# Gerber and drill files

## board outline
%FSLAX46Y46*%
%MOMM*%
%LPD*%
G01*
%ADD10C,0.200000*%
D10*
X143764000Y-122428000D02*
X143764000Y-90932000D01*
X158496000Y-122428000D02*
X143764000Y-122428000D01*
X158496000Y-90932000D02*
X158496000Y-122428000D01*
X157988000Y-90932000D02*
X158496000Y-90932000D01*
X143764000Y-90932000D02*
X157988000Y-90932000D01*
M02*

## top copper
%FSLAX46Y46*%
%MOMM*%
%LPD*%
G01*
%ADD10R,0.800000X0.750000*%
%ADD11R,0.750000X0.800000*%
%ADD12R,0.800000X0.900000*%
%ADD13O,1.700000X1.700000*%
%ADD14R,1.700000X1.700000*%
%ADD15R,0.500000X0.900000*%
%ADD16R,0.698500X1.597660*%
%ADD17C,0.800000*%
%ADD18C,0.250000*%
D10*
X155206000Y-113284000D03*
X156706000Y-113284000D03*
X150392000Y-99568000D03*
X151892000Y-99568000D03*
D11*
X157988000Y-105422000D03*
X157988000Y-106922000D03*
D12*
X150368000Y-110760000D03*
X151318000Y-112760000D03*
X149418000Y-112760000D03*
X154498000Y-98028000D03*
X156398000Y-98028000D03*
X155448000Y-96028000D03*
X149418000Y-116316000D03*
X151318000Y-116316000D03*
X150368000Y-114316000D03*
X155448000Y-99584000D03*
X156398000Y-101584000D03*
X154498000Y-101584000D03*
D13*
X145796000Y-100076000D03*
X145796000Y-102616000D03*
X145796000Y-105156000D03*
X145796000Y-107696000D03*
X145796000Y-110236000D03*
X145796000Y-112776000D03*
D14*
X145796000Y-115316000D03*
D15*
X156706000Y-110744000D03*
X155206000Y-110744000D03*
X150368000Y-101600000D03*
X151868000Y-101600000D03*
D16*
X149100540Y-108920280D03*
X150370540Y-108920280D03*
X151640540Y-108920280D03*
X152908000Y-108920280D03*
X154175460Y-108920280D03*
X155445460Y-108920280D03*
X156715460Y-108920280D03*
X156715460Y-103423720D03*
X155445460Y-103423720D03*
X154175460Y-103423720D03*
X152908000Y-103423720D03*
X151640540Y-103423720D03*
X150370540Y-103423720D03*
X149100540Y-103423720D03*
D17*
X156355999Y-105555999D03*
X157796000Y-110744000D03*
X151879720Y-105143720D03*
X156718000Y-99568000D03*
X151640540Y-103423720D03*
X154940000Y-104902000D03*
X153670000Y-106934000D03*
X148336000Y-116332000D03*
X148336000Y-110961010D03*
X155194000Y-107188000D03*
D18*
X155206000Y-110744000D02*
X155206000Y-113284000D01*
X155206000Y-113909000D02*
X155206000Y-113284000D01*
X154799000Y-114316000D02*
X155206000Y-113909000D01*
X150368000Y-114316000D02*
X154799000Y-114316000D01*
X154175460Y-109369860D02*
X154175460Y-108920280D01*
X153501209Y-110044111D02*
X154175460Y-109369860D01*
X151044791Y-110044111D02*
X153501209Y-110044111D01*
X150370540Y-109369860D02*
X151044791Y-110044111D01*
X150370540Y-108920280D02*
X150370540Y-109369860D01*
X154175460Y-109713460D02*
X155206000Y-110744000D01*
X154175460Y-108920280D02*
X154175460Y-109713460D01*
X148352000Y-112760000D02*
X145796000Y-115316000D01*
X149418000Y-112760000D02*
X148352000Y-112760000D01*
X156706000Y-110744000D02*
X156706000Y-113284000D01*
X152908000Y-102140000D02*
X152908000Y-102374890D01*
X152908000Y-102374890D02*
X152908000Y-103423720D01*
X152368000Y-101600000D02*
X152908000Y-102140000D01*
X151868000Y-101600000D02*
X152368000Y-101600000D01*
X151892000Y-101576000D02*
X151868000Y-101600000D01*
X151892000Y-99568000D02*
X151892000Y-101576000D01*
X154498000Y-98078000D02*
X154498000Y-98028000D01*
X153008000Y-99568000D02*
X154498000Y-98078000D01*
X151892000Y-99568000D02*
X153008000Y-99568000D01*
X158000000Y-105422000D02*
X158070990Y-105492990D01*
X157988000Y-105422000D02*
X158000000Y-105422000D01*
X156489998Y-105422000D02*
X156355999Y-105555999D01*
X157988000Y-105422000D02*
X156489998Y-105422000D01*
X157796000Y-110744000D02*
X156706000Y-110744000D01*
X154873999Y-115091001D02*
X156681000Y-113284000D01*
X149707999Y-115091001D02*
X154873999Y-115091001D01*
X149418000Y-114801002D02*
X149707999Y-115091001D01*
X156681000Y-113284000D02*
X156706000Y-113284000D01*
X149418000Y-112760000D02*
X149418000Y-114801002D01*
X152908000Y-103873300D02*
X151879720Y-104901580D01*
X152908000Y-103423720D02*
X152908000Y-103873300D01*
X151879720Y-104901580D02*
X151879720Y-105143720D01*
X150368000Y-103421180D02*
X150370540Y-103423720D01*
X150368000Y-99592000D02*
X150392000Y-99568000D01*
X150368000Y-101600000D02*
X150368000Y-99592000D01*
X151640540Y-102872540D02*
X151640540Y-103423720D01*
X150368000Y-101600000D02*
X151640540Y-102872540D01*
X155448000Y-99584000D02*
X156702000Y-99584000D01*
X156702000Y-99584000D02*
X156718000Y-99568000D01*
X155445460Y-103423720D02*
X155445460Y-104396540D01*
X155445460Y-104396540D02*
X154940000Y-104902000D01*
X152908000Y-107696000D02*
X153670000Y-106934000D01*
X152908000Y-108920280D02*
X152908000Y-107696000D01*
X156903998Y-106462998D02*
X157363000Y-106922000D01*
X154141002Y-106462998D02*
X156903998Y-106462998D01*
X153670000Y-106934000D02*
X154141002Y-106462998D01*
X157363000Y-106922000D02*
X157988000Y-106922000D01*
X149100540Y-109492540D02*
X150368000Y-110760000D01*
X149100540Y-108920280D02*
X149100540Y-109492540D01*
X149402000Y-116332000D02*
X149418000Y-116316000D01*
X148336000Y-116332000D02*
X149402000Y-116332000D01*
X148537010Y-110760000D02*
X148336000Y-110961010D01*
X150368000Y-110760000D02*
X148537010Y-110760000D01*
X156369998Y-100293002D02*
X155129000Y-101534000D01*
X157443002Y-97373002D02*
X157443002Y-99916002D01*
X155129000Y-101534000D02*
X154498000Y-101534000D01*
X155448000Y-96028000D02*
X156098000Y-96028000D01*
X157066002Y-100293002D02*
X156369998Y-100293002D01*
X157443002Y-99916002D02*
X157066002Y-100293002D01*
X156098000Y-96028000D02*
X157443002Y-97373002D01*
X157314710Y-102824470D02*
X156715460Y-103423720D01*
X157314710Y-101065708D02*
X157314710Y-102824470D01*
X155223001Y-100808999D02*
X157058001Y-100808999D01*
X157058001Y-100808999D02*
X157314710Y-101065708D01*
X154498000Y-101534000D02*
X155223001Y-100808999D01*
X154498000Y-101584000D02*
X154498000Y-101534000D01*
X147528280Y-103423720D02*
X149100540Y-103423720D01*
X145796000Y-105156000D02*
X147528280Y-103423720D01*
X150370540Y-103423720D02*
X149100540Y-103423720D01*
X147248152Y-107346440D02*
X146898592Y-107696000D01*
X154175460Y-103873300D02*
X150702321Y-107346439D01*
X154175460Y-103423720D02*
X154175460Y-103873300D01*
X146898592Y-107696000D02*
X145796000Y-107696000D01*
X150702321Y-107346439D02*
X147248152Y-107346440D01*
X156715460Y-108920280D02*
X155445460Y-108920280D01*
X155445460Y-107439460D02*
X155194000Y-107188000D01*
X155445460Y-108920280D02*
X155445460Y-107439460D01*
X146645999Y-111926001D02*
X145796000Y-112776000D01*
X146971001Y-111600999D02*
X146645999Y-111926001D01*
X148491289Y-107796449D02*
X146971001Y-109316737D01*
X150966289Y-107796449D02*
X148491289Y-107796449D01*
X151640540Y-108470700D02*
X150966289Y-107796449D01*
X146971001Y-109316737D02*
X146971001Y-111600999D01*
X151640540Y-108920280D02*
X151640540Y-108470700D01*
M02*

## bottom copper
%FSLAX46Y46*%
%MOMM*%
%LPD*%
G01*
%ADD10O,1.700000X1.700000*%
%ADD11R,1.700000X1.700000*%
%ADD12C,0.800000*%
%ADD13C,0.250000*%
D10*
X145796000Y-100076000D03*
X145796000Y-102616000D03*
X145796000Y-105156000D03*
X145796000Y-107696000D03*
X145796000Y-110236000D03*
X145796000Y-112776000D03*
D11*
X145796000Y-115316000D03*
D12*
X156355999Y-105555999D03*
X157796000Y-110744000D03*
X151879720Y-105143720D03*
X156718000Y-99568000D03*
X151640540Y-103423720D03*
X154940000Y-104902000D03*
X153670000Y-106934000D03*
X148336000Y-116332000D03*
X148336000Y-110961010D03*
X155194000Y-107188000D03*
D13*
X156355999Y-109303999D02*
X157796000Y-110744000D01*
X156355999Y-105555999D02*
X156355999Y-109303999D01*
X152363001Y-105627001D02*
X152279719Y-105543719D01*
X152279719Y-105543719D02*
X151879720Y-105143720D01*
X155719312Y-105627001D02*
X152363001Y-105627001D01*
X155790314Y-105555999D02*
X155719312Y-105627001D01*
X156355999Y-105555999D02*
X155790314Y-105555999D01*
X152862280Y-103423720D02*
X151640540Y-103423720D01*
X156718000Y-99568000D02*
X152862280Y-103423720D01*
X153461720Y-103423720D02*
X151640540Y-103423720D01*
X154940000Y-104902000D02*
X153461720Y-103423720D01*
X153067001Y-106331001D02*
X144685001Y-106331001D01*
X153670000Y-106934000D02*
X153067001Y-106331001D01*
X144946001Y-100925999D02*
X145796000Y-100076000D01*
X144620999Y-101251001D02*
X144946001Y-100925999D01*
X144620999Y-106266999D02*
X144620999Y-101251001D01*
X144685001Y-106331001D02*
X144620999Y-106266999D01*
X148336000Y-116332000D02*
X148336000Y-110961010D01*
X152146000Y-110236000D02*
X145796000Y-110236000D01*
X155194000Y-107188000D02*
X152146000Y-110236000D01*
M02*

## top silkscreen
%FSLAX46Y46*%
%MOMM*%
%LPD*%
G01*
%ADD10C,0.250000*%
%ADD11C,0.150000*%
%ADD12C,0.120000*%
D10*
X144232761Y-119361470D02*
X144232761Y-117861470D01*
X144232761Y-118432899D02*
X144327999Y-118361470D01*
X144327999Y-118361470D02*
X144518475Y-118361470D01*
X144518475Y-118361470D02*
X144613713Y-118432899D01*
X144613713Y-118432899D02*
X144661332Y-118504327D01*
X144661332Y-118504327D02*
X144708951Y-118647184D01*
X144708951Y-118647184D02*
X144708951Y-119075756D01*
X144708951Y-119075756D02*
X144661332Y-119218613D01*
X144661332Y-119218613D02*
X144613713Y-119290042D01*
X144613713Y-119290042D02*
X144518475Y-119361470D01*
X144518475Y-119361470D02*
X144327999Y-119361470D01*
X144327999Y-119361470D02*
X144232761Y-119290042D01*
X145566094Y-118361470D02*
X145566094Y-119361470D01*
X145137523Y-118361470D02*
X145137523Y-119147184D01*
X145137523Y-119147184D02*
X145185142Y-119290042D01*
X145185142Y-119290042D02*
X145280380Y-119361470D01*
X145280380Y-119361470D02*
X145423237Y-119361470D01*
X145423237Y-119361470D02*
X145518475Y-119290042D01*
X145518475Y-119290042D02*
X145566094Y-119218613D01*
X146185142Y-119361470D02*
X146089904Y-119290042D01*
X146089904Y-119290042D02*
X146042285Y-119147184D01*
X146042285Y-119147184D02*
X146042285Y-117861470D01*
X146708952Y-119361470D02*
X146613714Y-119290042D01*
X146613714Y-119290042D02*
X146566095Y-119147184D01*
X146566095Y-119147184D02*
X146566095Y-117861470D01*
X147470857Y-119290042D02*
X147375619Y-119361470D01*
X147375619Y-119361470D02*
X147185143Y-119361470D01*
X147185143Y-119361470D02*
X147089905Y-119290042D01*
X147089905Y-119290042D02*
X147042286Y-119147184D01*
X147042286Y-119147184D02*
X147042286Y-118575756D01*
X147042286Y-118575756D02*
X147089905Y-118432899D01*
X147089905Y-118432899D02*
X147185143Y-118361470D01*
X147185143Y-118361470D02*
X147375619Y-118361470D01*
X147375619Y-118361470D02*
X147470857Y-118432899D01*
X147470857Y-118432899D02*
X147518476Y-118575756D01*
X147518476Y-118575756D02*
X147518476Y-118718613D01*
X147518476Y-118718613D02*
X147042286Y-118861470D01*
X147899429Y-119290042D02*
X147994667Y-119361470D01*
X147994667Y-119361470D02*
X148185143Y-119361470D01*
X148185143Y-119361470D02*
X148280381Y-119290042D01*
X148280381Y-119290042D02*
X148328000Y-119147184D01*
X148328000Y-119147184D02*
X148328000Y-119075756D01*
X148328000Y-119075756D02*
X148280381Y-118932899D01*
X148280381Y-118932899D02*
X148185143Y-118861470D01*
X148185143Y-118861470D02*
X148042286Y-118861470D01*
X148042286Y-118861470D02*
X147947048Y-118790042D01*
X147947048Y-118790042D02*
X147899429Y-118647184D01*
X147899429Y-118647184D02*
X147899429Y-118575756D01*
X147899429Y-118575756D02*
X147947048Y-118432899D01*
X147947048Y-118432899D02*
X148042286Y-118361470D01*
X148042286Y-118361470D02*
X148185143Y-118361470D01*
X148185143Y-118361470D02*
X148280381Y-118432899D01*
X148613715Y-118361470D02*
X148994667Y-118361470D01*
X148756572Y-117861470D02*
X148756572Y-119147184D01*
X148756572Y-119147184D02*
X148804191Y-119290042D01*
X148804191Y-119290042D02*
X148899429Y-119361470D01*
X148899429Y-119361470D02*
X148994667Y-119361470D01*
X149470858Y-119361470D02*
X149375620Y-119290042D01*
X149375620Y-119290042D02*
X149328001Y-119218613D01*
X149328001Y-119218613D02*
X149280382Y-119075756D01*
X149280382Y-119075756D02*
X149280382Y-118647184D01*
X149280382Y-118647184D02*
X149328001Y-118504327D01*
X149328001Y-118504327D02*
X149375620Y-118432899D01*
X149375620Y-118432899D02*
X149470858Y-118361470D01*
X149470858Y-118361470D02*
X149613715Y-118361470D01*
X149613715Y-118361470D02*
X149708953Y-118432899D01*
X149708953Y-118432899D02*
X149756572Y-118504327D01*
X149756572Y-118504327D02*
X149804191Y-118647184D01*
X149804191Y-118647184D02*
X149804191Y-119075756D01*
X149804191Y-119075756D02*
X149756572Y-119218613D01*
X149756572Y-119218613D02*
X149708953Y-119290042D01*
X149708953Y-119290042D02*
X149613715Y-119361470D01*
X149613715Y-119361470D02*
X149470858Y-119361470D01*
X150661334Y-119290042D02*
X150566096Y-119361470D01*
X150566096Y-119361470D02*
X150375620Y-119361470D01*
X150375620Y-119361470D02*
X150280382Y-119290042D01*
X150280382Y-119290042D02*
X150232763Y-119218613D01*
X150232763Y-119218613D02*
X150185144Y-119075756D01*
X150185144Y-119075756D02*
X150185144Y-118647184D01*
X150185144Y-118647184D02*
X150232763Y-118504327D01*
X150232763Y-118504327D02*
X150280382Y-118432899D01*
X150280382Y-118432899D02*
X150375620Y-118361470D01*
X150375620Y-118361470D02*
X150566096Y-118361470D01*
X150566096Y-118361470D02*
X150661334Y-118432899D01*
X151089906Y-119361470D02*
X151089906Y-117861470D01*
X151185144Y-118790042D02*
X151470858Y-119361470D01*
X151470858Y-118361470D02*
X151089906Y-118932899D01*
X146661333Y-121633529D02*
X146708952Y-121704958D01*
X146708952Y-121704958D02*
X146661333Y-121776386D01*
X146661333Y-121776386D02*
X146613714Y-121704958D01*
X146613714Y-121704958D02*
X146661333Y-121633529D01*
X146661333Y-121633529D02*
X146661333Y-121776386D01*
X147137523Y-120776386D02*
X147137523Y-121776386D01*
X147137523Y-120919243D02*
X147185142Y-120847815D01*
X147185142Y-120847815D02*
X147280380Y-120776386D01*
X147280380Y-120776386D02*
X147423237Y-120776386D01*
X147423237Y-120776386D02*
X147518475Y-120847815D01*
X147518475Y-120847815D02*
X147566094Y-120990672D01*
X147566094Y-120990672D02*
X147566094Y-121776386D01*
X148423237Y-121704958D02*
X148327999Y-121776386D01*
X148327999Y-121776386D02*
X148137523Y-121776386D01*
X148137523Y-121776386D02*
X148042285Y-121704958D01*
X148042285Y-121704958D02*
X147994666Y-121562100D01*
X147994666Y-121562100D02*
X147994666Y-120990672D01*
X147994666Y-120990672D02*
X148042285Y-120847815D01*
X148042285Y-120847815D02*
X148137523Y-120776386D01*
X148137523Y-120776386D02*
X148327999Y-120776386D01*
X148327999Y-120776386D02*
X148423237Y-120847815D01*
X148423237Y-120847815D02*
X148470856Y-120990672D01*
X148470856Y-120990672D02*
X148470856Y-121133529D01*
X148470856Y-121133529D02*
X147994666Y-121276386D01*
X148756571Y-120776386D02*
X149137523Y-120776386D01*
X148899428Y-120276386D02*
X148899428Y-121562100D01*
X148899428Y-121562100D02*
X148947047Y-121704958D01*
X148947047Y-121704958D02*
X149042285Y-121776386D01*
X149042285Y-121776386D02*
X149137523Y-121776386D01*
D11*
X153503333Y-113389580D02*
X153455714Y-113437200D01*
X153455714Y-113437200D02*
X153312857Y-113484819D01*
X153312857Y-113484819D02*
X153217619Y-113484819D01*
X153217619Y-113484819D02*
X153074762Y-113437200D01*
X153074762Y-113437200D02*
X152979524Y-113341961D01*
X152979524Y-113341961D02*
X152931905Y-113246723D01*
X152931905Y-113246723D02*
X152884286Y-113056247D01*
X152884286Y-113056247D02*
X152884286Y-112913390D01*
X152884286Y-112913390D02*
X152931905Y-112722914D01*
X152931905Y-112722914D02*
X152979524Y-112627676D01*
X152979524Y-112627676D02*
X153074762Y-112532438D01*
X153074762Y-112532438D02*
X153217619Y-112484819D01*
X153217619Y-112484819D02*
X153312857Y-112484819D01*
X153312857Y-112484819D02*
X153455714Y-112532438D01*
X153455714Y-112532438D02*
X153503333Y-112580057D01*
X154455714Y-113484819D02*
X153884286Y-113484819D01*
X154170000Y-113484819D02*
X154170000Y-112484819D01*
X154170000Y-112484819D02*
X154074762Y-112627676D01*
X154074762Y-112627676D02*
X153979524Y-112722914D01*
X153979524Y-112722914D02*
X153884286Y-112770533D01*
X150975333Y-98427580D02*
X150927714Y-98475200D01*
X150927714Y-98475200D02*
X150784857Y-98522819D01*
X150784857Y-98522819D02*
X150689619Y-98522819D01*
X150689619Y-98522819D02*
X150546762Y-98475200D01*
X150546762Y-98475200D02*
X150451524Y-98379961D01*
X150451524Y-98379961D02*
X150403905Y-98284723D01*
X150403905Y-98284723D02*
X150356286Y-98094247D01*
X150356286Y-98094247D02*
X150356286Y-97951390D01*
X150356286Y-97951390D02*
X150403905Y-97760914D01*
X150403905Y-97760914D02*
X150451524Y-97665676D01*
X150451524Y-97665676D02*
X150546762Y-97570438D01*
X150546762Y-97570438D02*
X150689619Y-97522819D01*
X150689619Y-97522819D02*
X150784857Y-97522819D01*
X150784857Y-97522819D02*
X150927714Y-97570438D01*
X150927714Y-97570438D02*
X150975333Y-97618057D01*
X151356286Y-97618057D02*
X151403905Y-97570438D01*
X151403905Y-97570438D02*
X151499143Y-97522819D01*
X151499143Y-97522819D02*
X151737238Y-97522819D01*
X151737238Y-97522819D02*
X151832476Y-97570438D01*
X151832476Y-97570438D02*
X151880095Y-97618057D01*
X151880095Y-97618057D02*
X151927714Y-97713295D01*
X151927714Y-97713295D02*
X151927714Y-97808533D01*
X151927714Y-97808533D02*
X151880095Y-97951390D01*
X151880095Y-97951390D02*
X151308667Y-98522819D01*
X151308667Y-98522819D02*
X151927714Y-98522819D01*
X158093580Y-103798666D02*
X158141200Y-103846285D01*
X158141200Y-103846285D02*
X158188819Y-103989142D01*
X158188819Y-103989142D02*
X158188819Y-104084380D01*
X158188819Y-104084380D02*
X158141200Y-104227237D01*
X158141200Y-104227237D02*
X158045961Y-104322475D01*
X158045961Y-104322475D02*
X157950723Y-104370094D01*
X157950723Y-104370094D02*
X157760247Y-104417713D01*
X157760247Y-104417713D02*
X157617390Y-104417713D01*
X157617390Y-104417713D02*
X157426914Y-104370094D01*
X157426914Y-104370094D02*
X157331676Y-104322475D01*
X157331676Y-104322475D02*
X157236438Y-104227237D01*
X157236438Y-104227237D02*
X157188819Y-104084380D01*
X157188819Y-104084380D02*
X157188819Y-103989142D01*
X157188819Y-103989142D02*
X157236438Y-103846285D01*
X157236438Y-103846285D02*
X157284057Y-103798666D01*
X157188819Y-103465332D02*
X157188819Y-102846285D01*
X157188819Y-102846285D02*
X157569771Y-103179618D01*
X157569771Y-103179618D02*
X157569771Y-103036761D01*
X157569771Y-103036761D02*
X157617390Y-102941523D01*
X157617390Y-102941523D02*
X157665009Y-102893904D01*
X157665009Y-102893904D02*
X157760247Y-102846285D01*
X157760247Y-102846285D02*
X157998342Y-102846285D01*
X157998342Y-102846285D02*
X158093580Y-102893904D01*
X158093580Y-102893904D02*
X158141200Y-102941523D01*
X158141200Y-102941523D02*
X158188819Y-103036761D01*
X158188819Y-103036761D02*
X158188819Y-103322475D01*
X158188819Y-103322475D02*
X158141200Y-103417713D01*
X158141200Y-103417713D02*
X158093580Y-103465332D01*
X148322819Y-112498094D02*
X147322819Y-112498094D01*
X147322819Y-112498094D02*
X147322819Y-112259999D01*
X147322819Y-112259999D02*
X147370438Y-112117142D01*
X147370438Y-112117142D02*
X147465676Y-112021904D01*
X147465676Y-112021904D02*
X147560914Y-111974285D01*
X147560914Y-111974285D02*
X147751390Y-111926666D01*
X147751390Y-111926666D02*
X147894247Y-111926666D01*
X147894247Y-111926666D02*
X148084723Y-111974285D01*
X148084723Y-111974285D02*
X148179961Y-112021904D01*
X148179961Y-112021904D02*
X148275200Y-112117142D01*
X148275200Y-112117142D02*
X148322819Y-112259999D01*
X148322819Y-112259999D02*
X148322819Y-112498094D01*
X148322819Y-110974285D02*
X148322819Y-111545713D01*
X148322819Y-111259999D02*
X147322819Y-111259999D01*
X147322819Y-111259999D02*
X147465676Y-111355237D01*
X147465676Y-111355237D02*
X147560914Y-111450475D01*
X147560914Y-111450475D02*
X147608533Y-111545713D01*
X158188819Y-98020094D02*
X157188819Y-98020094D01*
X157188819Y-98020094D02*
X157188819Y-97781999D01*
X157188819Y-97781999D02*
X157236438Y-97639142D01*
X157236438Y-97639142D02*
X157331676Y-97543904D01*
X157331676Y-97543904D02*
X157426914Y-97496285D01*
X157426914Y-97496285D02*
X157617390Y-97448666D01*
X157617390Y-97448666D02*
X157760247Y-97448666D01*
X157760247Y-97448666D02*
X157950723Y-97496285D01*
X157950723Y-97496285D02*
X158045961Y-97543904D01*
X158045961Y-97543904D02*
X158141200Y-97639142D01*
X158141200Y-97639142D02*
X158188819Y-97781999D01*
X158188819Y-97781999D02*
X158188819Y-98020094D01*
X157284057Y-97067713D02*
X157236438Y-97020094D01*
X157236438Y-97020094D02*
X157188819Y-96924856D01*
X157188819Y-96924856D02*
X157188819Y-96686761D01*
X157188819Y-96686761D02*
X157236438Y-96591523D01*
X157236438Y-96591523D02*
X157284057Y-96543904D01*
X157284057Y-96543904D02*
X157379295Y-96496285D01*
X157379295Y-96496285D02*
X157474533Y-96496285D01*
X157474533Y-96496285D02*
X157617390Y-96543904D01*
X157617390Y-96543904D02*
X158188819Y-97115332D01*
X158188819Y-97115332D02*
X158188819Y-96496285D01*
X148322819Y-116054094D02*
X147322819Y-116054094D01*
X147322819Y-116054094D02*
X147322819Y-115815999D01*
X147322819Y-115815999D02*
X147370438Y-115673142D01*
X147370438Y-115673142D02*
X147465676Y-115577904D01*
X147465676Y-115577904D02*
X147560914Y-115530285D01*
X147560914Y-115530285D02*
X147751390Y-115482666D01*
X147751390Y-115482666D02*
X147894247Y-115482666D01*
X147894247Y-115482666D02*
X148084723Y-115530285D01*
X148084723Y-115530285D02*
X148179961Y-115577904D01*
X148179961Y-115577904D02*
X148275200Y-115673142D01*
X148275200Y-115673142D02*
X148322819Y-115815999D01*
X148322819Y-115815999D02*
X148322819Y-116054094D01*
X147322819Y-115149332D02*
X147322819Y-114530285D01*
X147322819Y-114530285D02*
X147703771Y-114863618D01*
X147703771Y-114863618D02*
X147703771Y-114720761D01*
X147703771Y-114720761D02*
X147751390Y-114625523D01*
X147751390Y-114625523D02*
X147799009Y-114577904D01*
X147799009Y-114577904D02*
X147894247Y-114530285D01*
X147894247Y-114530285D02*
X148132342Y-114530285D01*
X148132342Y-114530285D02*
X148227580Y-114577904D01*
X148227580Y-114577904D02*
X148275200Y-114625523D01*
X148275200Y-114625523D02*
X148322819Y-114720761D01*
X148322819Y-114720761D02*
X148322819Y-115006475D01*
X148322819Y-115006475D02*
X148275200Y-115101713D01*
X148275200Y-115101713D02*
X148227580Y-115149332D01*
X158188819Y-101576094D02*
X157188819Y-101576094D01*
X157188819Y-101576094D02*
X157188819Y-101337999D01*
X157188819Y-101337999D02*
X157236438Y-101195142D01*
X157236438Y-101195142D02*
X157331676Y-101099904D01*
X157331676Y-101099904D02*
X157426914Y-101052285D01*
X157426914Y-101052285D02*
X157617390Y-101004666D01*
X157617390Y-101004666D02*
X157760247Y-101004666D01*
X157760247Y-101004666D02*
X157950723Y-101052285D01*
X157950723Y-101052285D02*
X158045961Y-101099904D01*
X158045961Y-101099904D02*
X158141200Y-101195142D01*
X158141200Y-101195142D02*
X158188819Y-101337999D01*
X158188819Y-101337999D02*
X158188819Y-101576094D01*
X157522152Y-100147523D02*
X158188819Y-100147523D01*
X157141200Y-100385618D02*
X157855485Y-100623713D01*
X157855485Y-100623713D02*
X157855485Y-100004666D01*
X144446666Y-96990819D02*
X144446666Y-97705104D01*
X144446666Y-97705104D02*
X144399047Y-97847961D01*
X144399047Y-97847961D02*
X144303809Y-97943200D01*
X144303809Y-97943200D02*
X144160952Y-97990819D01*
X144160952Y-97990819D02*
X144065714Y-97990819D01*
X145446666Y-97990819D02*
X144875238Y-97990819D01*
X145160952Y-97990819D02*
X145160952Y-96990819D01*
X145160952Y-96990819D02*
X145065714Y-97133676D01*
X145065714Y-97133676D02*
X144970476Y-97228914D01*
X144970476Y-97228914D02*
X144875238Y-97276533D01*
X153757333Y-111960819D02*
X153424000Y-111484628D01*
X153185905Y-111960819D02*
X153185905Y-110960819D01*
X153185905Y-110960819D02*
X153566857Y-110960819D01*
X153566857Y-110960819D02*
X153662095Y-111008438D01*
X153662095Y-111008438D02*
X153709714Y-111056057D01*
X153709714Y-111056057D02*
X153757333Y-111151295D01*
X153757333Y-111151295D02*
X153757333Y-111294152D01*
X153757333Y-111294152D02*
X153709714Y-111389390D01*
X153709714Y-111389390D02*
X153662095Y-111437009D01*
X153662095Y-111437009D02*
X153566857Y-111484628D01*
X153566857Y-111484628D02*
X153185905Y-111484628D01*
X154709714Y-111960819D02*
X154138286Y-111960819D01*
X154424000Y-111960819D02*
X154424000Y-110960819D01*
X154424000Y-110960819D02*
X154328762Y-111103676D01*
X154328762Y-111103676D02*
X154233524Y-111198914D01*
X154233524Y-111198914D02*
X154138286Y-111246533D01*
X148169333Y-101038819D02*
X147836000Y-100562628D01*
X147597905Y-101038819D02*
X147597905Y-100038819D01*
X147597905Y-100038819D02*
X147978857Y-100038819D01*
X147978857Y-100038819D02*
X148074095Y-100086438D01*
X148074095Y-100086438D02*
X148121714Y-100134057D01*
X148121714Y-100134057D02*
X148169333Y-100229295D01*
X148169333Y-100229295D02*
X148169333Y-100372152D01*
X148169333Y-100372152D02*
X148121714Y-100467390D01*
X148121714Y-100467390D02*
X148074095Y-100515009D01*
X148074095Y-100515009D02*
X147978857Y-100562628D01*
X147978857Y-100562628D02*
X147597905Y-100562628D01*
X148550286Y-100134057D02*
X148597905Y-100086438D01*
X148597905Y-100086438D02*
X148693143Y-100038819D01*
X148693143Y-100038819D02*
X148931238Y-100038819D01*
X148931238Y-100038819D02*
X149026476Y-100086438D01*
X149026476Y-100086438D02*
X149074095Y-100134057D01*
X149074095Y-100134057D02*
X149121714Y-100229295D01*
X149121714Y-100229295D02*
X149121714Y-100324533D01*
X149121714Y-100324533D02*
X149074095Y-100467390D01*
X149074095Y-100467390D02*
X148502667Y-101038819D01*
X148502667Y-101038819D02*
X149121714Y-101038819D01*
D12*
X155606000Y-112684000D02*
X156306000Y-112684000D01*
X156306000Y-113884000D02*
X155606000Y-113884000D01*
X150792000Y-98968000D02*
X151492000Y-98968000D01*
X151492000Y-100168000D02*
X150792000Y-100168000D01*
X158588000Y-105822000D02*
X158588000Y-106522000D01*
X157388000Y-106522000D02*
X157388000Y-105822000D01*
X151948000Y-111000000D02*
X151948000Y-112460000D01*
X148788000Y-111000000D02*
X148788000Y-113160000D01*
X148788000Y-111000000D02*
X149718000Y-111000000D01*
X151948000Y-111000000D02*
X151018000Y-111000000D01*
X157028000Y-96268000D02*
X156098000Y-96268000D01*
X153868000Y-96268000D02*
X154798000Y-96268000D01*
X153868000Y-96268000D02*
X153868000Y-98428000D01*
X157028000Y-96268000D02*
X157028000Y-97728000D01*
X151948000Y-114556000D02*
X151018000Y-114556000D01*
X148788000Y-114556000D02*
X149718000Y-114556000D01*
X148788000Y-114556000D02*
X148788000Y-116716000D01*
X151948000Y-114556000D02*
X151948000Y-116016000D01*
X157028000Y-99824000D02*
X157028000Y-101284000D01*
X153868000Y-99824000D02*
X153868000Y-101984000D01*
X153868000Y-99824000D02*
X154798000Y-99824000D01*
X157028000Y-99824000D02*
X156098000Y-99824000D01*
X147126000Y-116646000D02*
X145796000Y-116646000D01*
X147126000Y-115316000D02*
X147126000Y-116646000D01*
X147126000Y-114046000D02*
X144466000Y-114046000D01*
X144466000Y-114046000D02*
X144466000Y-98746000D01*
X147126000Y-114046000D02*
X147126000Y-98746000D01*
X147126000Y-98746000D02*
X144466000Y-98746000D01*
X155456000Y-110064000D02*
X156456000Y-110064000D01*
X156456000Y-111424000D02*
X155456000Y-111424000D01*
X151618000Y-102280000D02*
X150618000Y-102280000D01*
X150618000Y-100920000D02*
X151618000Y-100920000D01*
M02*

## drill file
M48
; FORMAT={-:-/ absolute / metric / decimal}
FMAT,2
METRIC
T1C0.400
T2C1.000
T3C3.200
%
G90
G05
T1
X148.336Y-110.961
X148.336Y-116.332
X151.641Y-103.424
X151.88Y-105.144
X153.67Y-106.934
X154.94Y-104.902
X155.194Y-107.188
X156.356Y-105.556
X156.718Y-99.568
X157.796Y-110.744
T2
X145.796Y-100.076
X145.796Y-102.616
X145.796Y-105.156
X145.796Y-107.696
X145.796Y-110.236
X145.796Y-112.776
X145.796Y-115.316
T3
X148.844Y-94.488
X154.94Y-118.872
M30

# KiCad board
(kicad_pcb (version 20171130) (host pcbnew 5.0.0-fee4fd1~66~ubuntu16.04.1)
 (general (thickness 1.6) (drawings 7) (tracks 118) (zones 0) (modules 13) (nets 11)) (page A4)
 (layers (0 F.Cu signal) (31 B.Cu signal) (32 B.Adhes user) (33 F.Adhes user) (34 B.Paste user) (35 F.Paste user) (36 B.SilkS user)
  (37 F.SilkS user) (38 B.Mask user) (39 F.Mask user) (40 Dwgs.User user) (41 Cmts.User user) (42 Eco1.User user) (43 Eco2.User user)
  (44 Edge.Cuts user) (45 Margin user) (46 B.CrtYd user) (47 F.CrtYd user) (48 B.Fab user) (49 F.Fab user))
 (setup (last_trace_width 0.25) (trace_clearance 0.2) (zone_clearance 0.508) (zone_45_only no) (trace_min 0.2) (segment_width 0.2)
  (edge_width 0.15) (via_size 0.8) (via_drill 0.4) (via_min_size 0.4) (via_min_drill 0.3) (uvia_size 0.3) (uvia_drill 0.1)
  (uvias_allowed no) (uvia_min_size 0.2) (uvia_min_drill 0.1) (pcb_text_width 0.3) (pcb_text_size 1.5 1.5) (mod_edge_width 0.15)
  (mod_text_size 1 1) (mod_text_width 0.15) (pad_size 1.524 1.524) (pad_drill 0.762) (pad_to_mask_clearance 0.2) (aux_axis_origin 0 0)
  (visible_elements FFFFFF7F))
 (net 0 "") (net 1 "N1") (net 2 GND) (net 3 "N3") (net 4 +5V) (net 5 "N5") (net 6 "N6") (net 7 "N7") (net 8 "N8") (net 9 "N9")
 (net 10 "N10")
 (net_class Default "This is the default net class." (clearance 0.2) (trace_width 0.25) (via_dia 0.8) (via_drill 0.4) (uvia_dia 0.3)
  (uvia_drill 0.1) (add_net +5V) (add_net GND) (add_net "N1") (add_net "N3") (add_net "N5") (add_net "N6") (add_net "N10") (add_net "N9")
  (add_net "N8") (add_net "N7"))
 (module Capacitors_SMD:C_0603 (layer F.Cu) (at 155.956 113.284)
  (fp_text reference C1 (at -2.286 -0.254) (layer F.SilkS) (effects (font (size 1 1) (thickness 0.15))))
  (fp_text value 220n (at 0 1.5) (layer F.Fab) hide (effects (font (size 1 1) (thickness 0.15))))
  (fp_line (start -0.35 -0.6) (end 0.35 -0.6) (layer F.SilkS) (width 0.12))
  (fp_line (start 0.35 0.6) (end -0.35 0.6) (layer F.SilkS) (width 0.12))
  (pad 1 smd rect (at -0.75 0) (size 0.8 0.75) (layers F.Cu F.Paste F.Mask) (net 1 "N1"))
  (pad 2 smd rect (at 0.75 0) (size 0.8 0.75) (layers F.Cu F.Paste F.Mask) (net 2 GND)))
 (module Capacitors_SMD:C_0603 (layer F.Cu) (at 151.142 99.568)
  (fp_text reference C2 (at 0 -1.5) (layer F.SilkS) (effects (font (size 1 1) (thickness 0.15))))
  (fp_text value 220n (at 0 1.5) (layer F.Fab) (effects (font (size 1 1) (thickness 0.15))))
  (fp_line (start -0.35 -0.6) (end 0.35 -0.6) (layer F.SilkS) (width 0.12))
  (fp_line (start 0.35 0.6) (end -0.35 0.6) (layer F.SilkS) (width 0.12))
  (pad 1 smd rect (at -0.75 0) (size 0.8 0.75) (layers F.Cu F.Paste F.Mask) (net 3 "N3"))
  (pad 2 smd rect (at 0.75 0) (size 0.8 0.75) (layers F.Cu F.Paste F.Mask) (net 2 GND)))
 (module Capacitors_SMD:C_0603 (layer F.Cu) (at 157.988 106.172 90)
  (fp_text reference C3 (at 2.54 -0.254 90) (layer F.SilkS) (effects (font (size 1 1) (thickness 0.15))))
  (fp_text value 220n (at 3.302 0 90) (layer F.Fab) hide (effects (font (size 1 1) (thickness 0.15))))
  (fp_line (start 0.35 0.6) (end -0.35 0.6) (layer F.SilkS) (width 0.12))
  (fp_line (start -0.35 -0.6) (end 0.35 -0.6) (layer F.SilkS) (width 0.12))
  (pad 2 smd rect (at 0.75 0 90) (size 0.8 0.75) (layers F.Cu F.Paste F.Mask) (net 2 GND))
  (pad 1 smd rect (at -0.75 0 90) (size 0.8 0.75) (layers F.Cu F.Paste F.Mask) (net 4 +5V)))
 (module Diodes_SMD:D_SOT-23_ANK (layer F.Cu) (at 150.368 111.76 90)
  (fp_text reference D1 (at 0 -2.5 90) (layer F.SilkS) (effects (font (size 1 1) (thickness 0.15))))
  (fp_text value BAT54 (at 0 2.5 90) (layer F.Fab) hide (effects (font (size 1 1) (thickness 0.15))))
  (fp_line (start 0.76 1.58) (end -0.7 1.58) (layer F.SilkS) (width 0.12))
  (fp_line (start 0.76 -1.58) (end -1.4 -1.58) (layer F.SilkS) (width 0.12))
  (fp_line (start 0.76 -1.58) (end 0.76 -0.65) (layer F.SilkS) (width 0.12))
  (fp_line (start 0.76 1.58) (end 0.76 0.65) (layer F.SilkS) (width 0.12))
  (pad 1 smd rect (at 1 0 90) (size 0.9 0.8) (layers F.Cu F.Paste F.Mask) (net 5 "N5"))
  (pad "" smd rect (at -1 0.95 90) (size 0.9 0.8) (layers F.Cu F.Paste F.Mask))
  (pad 2 smd rect (at -1 -0.95 90) (size 0.9 0.8) (layers F.Cu F.Paste F.Mask) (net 2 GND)))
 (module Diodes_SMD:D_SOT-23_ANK (layer F.Cu) (at 155.448 97.028 90)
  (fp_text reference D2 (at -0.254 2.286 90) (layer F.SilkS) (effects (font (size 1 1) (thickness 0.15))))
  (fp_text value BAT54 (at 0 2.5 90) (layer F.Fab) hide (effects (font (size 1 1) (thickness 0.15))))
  (fp_line (start 0.76 1.58) (end 0.76 0.65) (layer F.SilkS) (width 0.12))
  (fp_line (start 0.76 -1.58) (end 0.76 -0.65) (layer F.SilkS) (width 0.12))
  (fp_line (start 0.76 -1.58) (end -1.4 -1.58) (layer F.SilkS) (width 0.12))
  (fp_line (start 0.76 1.58) (end -0.7 1.58) (layer F.SilkS) (width 0.12))
  (pad 2 smd rect (at -1 -0.95 90) (size 0.9 0.8) (layers F.Cu F.Paste F.Mask) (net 2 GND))
  (pad "" smd rect (at -1 0.95 90) (size 0.9 0.8) (layers F.Cu F.Paste F.Mask))
  (pad 1 smd rect (at 1 0 90) (size 0.9 0.8) (layers F.Cu F.Paste F.Mask) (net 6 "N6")))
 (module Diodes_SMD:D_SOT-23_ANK (layer F.Cu) (at 150.368 115.316 90)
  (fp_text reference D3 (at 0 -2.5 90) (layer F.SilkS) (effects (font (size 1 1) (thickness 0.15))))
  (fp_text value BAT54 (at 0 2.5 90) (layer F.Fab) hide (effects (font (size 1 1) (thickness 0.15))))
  (fp_line (start 0.76 1.58) (end 0.76 0.65) (layer F.SilkS) (width 0.12))
  (fp_line (start 0.76 -1.58) (end 0.76 -0.65) (layer F.SilkS) (width 0.12))
  (fp_line (start 0.76 -1.58) (end -1.4 -1.58) (layer F.SilkS) (width 0.12))
  (fp_line (start 0.76 1.58) (end -0.7 1.58) (layer F.SilkS) (width 0.12))
  (pad 2 smd rect (at -1 -0.95 90) (size 0.9 0.8) (layers F.Cu F.Paste F.Mask) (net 5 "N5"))
  (pad "" smd rect (at -1 0.95 90) (size 0.9 0.8) (layers F.Cu F.Paste F.Mask))
  (pad 1 smd rect (at 1 0 90) (size 0.9 0.8) (layers F.Cu F.Paste F.Mask) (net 1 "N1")))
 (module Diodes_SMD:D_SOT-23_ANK (layer F.Cu) (at 155.448 100.584 90)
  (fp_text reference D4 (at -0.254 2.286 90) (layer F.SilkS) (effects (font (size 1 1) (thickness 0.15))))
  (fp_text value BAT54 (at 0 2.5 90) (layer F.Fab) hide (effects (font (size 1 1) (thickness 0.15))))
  (fp_line (start 0.76 1.58) (end -0.7 1.58) (layer F.SilkS) (width 0.12))
  (fp_line (start 0.76 -1.58) (end -1.4 -1.58) (layer F.SilkS) (width 0.12))
  (fp_line (start 0.76 -1.58) (end 0.76 -0.65) (layer F.SilkS) (width 0.12))
  (fp_line (start 0.76 1.58) (end 0.76 0.65) (layer F.SilkS) (width 0.12))
  (pad 1 smd rect (at 1 0 90) (size 0.9 0.8) (layers F.Cu F.Paste F.Mask) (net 3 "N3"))
  (pad "" smd rect (at -1 0.95 90) (size 0.9 0.8) (layers F.Cu F.Paste F.Mask))
  (pad 2 smd rect (at -1 -0.95 90) (size 0.9 0.8) (layers F.Cu F.Paste F.Mask) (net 6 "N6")))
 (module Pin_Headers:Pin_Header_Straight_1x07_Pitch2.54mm (layer F.Cu) (at 145.796 115.316 180)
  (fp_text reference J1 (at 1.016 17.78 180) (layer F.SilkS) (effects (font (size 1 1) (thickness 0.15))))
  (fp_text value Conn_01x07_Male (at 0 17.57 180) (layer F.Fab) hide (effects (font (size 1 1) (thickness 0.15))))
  (fp_line (start -1.33 -1.33) (end 0 -1.33) (layer F.SilkS) (width 0.12))
  (fp_line (start -1.33 0) (end -1.33 -1.33) (layer F.SilkS) (width 0.12))
  (fp_line (start -1.33 1.27) (end 1.33 1.27) (layer F.SilkS) (width 0.12))
  (fp_line (start 1.33 1.27) (end 1.33 16.57) (layer F.SilkS) (width 0.12))
  (fp_line (start -1.33 1.27) (end -1.33 16.57) (layer F.SilkS) (width 0.12))
  (fp_line (start -1.33 16.57) (end 1.33 16.57) (layer F.SilkS) (width 0.12))
  (pad 7 thru_hole oval (at 0 15.24 180) (size 1.7 1.7) (drill 1) (layers *.Cu *.Mask) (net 4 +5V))
  (pad 6 thru_hole oval (at 0 12.7 180) (size 1.7 1.7) (drill 1) (layers *.Cu *.Mask))
  (pad 5 thru_hole oval (at 0 10.16 180) (size 1.7 1.7) (drill 1) (layers *.Cu *.Mask) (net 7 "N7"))
  (pad 4 thru_hole oval (at 0 7.62 180) (size 1.7 1.7) (drill 1) (layers *.Cu *.Mask) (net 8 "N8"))
  (pad 3 thru_hole oval (at 0 5.08 180) (size 1.7 1.7) (drill 1) (layers *.Cu *.Mask) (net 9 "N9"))
  (pad 2 thru_hole oval (at 0 2.54 180) (size 1.7 1.7) (drill 1) (layers *.Cu *.Mask) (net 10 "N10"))
  (pad 1 thru_hole rect (at 0 0 180) (size 1.7 1.7) (drill 1) (layers *.Cu *.Mask) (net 2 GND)))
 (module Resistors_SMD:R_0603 (layer F.Cu) (at 155.956 110.744)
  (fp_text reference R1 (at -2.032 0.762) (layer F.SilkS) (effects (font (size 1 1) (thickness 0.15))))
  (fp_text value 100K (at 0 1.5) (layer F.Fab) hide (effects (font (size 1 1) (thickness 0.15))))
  (fp_line (start -0.5 -0.68) (end 0.5 -0.68) (layer F.SilkS) (width 0.12))
  (fp_line (start 0.5 0.68) (end -0.5 0.68) (layer F.SilkS) (width 0.12))
  (pad 2 smd rect (at 0.75 0) (size 0.5 0.9) (layers F.Cu F.Paste F.Mask) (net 2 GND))
  (pad 1 smd rect (at -0.75 0) (size 0.5 0.9) (layers F.Cu F.Paste F.Mask) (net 1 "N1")))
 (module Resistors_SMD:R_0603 (layer F.Cu) (at 151.118 101.6)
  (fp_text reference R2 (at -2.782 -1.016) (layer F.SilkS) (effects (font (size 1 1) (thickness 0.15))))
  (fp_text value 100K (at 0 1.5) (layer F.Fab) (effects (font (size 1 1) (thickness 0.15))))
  (fp_line (start 0.5 0.68) (end -0.5 0.68) (layer F.SilkS) (width 0.12))
  (fp_line (start -0.5 -0.68) (end 0.5 -0.68) (layer F.SilkS) (width 0.12))
  (pad 1 smd rect (at -0.75 0) (size 0.5 0.9) (layers F.Cu F.Paste F.Mask) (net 3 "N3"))
  (pad 2 smd rect (at 0.75 0) (size 0.5 0.9) (layers F.Cu F.Paste F.Mask) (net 2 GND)))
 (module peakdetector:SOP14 (layer F.Cu) (at 152.908 106.172)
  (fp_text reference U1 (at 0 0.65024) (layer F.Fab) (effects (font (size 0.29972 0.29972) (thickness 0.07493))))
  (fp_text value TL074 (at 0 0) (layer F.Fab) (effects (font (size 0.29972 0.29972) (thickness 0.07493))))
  (pad 1 smd rect (at -3.80746 2.74828 180) (size 0.6985 1.59766) (layers F.Cu F.Paste F.Mask) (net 5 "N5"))
  (pad 2 smd rect (at -2.53746 2.74828 180) (size 0.6985 1.59766) (layers F.Cu F.Paste F.Mask) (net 1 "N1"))
  (pad 3 smd rect (at -1.26746 2.74828 180) (size 0.6985 1.59766) (layers F.Cu F.Paste F.Mask) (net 10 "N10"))
  (pad 4 smd rect (at 0 2.74828 180) (size 0.6985 1.59766) (layers F.Cu F.Paste F.Mask) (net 4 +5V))
  (pad 5 smd rect (at 1.26746 2.74828 180) (size 0.6985 1.59766) (layers F.Cu F.Paste F.Mask) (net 1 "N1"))
  (pad 6 smd rect (at 2.53746 2.74828 180) (size 0.6985 1.59766) (layers F.Cu F.Paste F.Mask) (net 9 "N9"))
  (pad 7 smd rect (at 3.80746 2.74828 180) (size 0.6985 1.59766) (layers F.Cu F.Paste F.Mask) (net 9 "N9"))
  (pad 8 smd rect (at 3.80746 -2.74828) (size 0.6985 1.59766) (layers F.Cu F.Paste F.Mask) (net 6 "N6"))
  (pad 9 smd rect (at 2.53746 -2.74828) (size 0.6985 1.59766) (layers F.Cu F.Paste F.Mask) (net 3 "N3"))
  (pad 10 smd rect (at 1.26746 -2.74828) (size 0.6985 1.59766) (layers F.Cu F.Paste F.Mask) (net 8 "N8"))
  (pad 11 smd rect (at 0 -2.74828) (size 0.6985 1.59766) (layers F.Cu F.Paste F.Mask) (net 2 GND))
  (pad 12 smd rect (at -1.26746 -2.74828) (size 0.6985 1.59766) (layers F.Cu F.Paste F.Mask) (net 3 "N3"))
  (pad 13 smd rect (at -2.53746 -2.74828) (size 0.6985 1.59766) (layers F.Cu F.Paste F.Mask) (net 7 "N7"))
  (pad 14 smd rect (at -3.80746 -2.74828) (size 0.6985 1.59766) (layers F.Cu F.Paste F.Mask) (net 7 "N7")))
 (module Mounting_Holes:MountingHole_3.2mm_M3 (layer F.Cu) (at 154.94 118.872)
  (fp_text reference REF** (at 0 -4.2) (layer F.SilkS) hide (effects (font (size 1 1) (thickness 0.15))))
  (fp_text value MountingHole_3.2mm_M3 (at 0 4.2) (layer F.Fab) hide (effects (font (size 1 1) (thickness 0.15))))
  (pad 1 np_thru_hole circle (at 0 0) (size 3.2 3.2) (drill 3.2) (layers *.Cu *.Mask)))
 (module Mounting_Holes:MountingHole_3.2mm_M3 (layer F.Cu) (at 148.844 94.488)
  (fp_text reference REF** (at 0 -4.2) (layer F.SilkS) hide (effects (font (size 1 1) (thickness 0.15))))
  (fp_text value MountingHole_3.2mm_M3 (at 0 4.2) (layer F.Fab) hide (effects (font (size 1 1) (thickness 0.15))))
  (pad 1 np_thru_hole circle (at 0 0) (size 3.2 3.2) (drill 3.2) (layers *.Cu *.Mask)))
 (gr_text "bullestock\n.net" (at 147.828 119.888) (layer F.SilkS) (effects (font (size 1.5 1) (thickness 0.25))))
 (gr_line (start 143.764 122.428) (end 143.764 90.932) (layer Edge.Cuts) (width 0.2))
 (gr_line (start 158.496 122.428) (end 143.764 122.428) (layer Edge.Cuts) (width 0.2))
 (gr_line (start 158.496 90.932) (end 158.496 122.428) (layer Edge.Cuts) (width 0.2))
 (gr_line (start 157.988 90.932) (end 158.496 90.932) (layer Edge.Cuts) (width 0.2))
 (gr_line (start 143.764 90.932) (end 157.988 90.932) (layer Edge.Cuts) (width 0.2))
 (segment (start 155.206 110.744) (end 155.206 113.284) (width 0.25) (layer F.Cu) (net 1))
 (segment (start 155.206 113.909) (end 155.206 113.284) (width 0.25) (layer F.Cu) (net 1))
 (segment (start 154.799 114.316) (end 155.206 113.909) (width 0.25) (layer F.Cu) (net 1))
 (segment (start 150.368 114.316) (end 154.799 114.316) (width 0.25) (layer F.Cu) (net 1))
 (segment (start 154.17546 109.36986) (end 154.17546 108.92028) (width 0.25) (layer F.Cu) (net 1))
 (segment (start 153.501209 110.044111) (end 154.17546 109.36986) (width 0.25) (layer F.Cu) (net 1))
 (segment (start 151.044791 110.044111) (end 153.501209 110.044111) (width 0.25) (layer F.Cu) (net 1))
 (segment (start 150.37054 109.36986) (end 151.044791 110.044111) (width 0.25) (layer F.Cu) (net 1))
 (segment (start 150.37054 108.92028) (end 150.37054 109.36986) (width 0.25) (layer F.Cu) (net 1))
 (segment (start 154.17546 109.71346) (end 155.206 110.744) (width 0.25) (layer F.Cu) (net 1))
 (segment (start 154.17546 108.92028) (end 154.17546 109.71346) (width 0.25) (layer F.Cu) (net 1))
 (segment (start 148.352 112.76) (end 145.796 115.316) (width 0.25) (layer F.Cu) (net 2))
 (segment (start 149.418 112.76) (end 148.352 112.76) (width 0.25) (layer F.Cu) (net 2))
 (segment (start 156.706 110.744) (end 156.706 113.284) (width 0.25) (layer F.Cu) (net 2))
 (segment (start 152.908 102.14) (end 152.908 102.37489) (width 0.25) (layer F.Cu) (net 2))
 (segment (start 152.908 102.37489) (end 152.908 103.42372) (width 0.25) (layer F.Cu) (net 2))
 (segment (start 152.368 101.6) (end 152.908 102.14) (width 0.25) (layer F.Cu) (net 2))
 (segment (start 151.868 101.6) (end 152.368 101.6) (width 0.25) (layer F.Cu) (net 2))
 (segment (start 151.892 101.576) (end 151.868 101.6) (width 0.25) (layer F.Cu) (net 2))
 (segment (start 151.892 99.568) (end 151.892 101.576) (width 0.25) (layer F.Cu) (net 2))
 (segment (start 154.498 98.078) (end 154.498 98.028) (width 0.25) (layer F.Cu) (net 2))
 (segment (start 153.008 99.568) (end 154.498 98.078) (width 0.25) (layer F.Cu) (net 2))
 (segment (start 151.892 99.568) (end 153.008 99.568) (width 0.25) (layer F.Cu) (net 2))
 (via (at 156.355999 105.555999) (size 0.8) (drill 0.4) (layers F.Cu B.Cu) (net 2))
 (segment (start 158 105.422) (end 158.07099 105.49299) (width 0.25) (layer F.Cu) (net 2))
 (segment (start 157.988 105.422) (end 158 105.422) (width 0.25) (layer F.Cu) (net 2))
 (segment (start 156.489998 105.422) (end 156.355999 105.555999) (width 0.25) (layer F.Cu) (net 2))
 (segment (start 157.988 105.422) (end 156.489998 105.422) (width 0.25) (layer F.Cu) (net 2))
 (via (at 157.796 110.744) (size 0.8) (drill 0.4) (layers F.Cu B.Cu) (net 2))
 (segment (start 156.355999 109.303999) (end 157.796 110.744) (width 0.25) (layer B.Cu) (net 2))
 (segment (start 156.355999 105.555999) (end 156.355999 109.303999) (width 0.25) (layer B.Cu) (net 2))
 (segment (start 157.796 110.744) (end 156.706 110.744) (width 0.25) (layer F.Cu) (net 2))
 (segment (start 154.873999 115.091001) (end 156.681 113.284) (width 0.25) (layer F.Cu) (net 2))
 (segment (start 149.707999 115.091001) (end 154.873999 115.091001) (width 0.25) (layer F.Cu) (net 2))
 (segment (start 149.418 114.801002) (end 149.707999 115.091001) (width 0.25) (layer F.Cu) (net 2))
 (segment (start 156.681 113.284) (end 156.706 113.284) (width 0.25) (layer F.Cu) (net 2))
 (segment (start 149.418 112.76) (end 149.418 114.801002) (width 0.25) (layer F.Cu) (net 2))
 (segment (start 152.908 103.8733) (end 151.87972 104.90158) (width 0.25) (layer F.Cu) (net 2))
 (segment (start 152.908 103.42372) (end 152.908 103.8733) (width 0.25) (layer F.Cu) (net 2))
 (via (at 151.87972 105.14372) (size 0.8) (drill 0.4) (layers F.Cu B.Cu) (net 2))
 (segment (start 151.87972 104.90158) (end 151.87972 105.14372) (width 0.25) (layer F.Cu) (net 2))
 (segment (start 152.363001 105.627001) (end 152.279719 105.543719) (width 0.25) (layer B.Cu) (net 2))
 (segment (start 152.279719 105.543719) (end 151.87972 105.14372) (width 0.25) (layer B.Cu) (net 2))
 (segment (start 155.719312 105.627001) (end 152.363001 105.627001) (width 0.25) (layer B.Cu) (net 2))
 (segment (start 155.790314 105.555999) (end 155.719312 105.627001) (width 0.25) (layer B.Cu) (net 2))
 (segment (start 156.355999 105.555999) (end 155.790314 105.555999) (width 0.25) (layer B.Cu) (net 2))
 (segment (start 150.368 103.42118) (end 150.37054 103.42372) (width 0.25) (layer F.Cu) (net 7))
 (segment (start 150.368 99.592) (end 150.392 99.568) (width 0.25) (layer F.Cu) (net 3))
 (segment (start 150.368 101.6) (end 150.368 99.592) (width 0.25) (layer F.Cu) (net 3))
 (segment (start 151.64054 102.87254) (end 151.64054 103.42372) (width 0.25) (layer F.Cu) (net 3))
 (segment (start 150.368 101.6) (end 151.64054 102.87254) (width 0.25) (layer F.Cu) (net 3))
 (via (at 156.718 99.568) (size 0.8) (drill 0.4) (layers F.Cu B.Cu) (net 3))
 (segment (start 155.448 99.584) (end 156.702 99.584) (width 0.25) (layer F.Cu) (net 3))
 (segment (start 156.702 99.584) (end 156.718 99.568) (width 0.25) (layer F.Cu) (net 3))
 (via (at 151.64054 103.42372) (size 0.8) (drill 0.4) (layers F.Cu B.Cu) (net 3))
 (segment (start 152.86228 103.42372) (end 151.64054 103.42372) (width 0.25) (layer B.Cu) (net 3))
 (segment (start 156.718 99.568) (end 152.86228 103.42372) (width 0.25) (layer B.Cu) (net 3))
 (via (at 154.94 104.902) (size 0.8) (drill 0.4) (layers F.Cu B.Cu) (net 3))
 (segment (start 155.44546 103.42372) (end 155.44546 104.39654) (width 0.25) (layer F.Cu) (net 3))
 (segment (start 155.44546 104.39654) (end 154.94 104.902) (width 0.25) (layer F.Cu) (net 3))
 (segment (start 153.46172 103.42372) (end 151.64054 103.42372) (width 0.25) (layer B.Cu) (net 3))
 (segment (start 154.94 104.902) (end 153.46172 103.42372) (width 0.25) (layer B.Cu) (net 3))
 (segment (start 152.908 107.696) (end 153.67 106.934) (width 0.25) (layer F.Cu) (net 4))
 (via (at 153.67 106.934) (size 0.8) (drill 0.4) (layers F.Cu B.Cu) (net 4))
 (segment (start 152.908 108.92028) (end 152.908 107.696) (width 0.25) (layer F.Cu) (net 4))
 (segment (start 153.067001 106.331001) (end 144.685001 106.331001) (width 0.25) (layer B.Cu) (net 4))
 (segment (start 153.67 106.934) (end 153.067001 106.331001) (width 0.25) (layer B.Cu) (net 4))
 (segment (start 144.946001 100.925999) (end 145.796 100.076) (width 0.25) (layer B.Cu) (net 4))
 (segment (start 144.620999 101.251001) (end 144.946001 100.925999) (width 0.25) (layer B.Cu) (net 4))
 (segment (start 144.620999 106.266999) (end 144.620999 101.251001) (width 0.25) (layer B.Cu) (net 4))
 (segment (start 144.685001 106.331001) (end 144.620999 106.266999) (width 0.25) (layer B.Cu) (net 4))
 (segment (start 156.903998 106.462998) (end 157.363 106.922) (width 0.25) (layer F.Cu) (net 4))
 (segment (start 154.141002 106.462998) (end 156.903998 106.462998) (width 0.25) (layer F.Cu) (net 4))
 (segment (start 153.67 106.934) (end 154.141002 106.462998) (width 0.25) (layer F.Cu) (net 4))
 (segment (start 157.363 106.922) (end 157.988 106.922) (width 0.25) (layer F.Cu) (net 4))
 (segment (start 149.10054 109.49254) (end 150.368 110.76) (width 0.25) (layer F.Cu) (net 5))
 (segment (start 149.10054 108.92028) (end 149.10054 109.49254) (width 0.25) (layer F.Cu) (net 5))
 (via (at 148.336 116.332) (size 0.8) (drill 0.4) (layers F.Cu B.Cu) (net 5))
 (segment (start 149.402 116.332) (end 149.418 116.316) (width 0.25) (layer F.Cu) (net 5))
 (segment (start 148.336 116.332) (end 149.402 116.332) (width 0.25) (layer F.Cu) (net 5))
 (segment (start 148.53701 110.76) (end 148.336 110.96101) (width 0.25) (layer F.Cu) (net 5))
 (segment (start 150.368 110.76) (end 148.53701 110.76) (width 0.25) (layer F.Cu) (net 5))
 (segment (start 148.336 116.332) (end 148.336 110.96101) (width 0.25) (layer B.Cu) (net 5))
 (via (at 148.336 110.96101) (size 0.8) (drill 0.4) (layers F.Cu B.Cu) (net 5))
 (segment (start 156.369998 100.293002) (end 155.129 101.534) (width 0.25) (layer F.Cu) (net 6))
 (segment (start 157.443002 97.373002) (end 157.443002 99.916002) (width 0.25) (layer F.Cu) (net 6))
 (segment (start 155.129 101.534) (end 154.498 101.534) (width 0.25) (layer F.Cu) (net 6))
 (segment (start 155.448 96.028) (end 156.098 96.028) (width 0.25) (layer F.Cu) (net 6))
 (segment (start 157.066002 100.293002) (end 156.369998 100.293002) (width 0.25) (layer F.Cu) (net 6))
 (segment (start 157.443002 99.916002) (end 157.066002 100.293002) (width 0.25) (layer F.Cu) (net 6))
 (segment (start 156.098 96.028) (end 157.443002 97.373002) (width 0.25) (layer F.Cu) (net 6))
 (segment (start 157.31471 102.82447) (end 156.71546 103.42372) (width 0.25) (layer F.Cu) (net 6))
 (segment (start 157.31471 101.065708) (end 157.31471 102.82447) (width 0.25) (layer F.Cu) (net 6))
 (segment (start 155.223001 100.808999) (end 157.058001 100.808999) (width 0.25) (layer F.Cu) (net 6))
 (segment (start 157.058001 100.808999) (end 157.31471 101.065708) (width 0.25) (layer F.Cu) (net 6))
 (segment (start 154.498 101.534) (end 155.223001 100.808999) (width 0.25) (layer F.Cu) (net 6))
 (segment (start 154.498 101.584) (end 154.498 101.534) (width 0.25) (layer F.Cu) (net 6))
 (segment (start 147.52828 103.42372) (end 149.10054 103.42372) (width 0.25) (layer F.Cu) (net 7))
 (segment (start 145.796 105.156) (end 147.52828 103.42372) (width 0.25) (layer F.Cu) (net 7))
 (segment (start 150.37054 103.42372) (end 149.10054 103.42372) (width 0.25) (layer F.Cu) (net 7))
 (segment (start 147.248152 107.34644) (end 146.898592 107.696) (width 0.25) (layer F.Cu) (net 8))
 (segment (start 154.17546 103.8733) (end 150.702321 107.346439) (width 0.25) (layer F.Cu) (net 8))
 (segment (start 154.17546 103.42372) (end 154.17546 103.8733) (width 0.25) (layer F.Cu) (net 8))
 (segment (start 146.898592 107.696) (end 145.796 107.696) (width 0.25) (layer F.Cu) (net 8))
 (segment (start 150.702321 107.346439) (end 147.248152 107.34644) (width 0.25) (layer F.Cu) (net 8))
 (segment (start 156.71546 108.92028) (end 155.44546 108.92028) (width 0.25) (layer F.Cu) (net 9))
 (segment (start 155.44546 107.43946) (end 155.194 107.188) (width 0.25) (layer F.Cu) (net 9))
 (via (at 155.194 107.188) (size 0.8) (drill 0.4) (layers F.Cu B.Cu) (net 9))
 (segment (start 155.44546 108.92028) (end 155.44546 107.43946) (width 0.25) (layer F.Cu) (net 9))
 (segment (start 152.146 110.236) (end 145.796 110.236) (width 0.25) (layer B.Cu) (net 9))
 (segment (start 155.194 107.188) (end 152.146 110.236) (width 0.25) (layer B.Cu) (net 9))
 (segment (start 146.645999 111.926001) (end 145.796 112.776) (width 0.25) (layer F.Cu) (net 10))
 (segment (start 146.971001 111.600999) (end 146.645999 111.926001) (width 0.25) (layer F.Cu) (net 10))
 (segment (start 148.491289 107.796449) (end 146.971001 109.316737) (width 0.25) (layer F.Cu) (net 10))
 (segment (start 150.966289 107.796449) (end 148.491289 107.796449) (width 0.25) (layer F.Cu) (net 10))
 (segment (start 151.64054 108.4707) (end 150.966289 107.796449) (width 0.25) (layer F.Cu) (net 10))
 (segment (start 146.971001 109.316737) (end 146.971001 111.600999) (width 0.25) (layer F.Cu) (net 10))
 (segment (start 151.64054 108.92028) (end 151.64054 108.4707) (width 0.25) (layer F.Cu) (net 10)))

